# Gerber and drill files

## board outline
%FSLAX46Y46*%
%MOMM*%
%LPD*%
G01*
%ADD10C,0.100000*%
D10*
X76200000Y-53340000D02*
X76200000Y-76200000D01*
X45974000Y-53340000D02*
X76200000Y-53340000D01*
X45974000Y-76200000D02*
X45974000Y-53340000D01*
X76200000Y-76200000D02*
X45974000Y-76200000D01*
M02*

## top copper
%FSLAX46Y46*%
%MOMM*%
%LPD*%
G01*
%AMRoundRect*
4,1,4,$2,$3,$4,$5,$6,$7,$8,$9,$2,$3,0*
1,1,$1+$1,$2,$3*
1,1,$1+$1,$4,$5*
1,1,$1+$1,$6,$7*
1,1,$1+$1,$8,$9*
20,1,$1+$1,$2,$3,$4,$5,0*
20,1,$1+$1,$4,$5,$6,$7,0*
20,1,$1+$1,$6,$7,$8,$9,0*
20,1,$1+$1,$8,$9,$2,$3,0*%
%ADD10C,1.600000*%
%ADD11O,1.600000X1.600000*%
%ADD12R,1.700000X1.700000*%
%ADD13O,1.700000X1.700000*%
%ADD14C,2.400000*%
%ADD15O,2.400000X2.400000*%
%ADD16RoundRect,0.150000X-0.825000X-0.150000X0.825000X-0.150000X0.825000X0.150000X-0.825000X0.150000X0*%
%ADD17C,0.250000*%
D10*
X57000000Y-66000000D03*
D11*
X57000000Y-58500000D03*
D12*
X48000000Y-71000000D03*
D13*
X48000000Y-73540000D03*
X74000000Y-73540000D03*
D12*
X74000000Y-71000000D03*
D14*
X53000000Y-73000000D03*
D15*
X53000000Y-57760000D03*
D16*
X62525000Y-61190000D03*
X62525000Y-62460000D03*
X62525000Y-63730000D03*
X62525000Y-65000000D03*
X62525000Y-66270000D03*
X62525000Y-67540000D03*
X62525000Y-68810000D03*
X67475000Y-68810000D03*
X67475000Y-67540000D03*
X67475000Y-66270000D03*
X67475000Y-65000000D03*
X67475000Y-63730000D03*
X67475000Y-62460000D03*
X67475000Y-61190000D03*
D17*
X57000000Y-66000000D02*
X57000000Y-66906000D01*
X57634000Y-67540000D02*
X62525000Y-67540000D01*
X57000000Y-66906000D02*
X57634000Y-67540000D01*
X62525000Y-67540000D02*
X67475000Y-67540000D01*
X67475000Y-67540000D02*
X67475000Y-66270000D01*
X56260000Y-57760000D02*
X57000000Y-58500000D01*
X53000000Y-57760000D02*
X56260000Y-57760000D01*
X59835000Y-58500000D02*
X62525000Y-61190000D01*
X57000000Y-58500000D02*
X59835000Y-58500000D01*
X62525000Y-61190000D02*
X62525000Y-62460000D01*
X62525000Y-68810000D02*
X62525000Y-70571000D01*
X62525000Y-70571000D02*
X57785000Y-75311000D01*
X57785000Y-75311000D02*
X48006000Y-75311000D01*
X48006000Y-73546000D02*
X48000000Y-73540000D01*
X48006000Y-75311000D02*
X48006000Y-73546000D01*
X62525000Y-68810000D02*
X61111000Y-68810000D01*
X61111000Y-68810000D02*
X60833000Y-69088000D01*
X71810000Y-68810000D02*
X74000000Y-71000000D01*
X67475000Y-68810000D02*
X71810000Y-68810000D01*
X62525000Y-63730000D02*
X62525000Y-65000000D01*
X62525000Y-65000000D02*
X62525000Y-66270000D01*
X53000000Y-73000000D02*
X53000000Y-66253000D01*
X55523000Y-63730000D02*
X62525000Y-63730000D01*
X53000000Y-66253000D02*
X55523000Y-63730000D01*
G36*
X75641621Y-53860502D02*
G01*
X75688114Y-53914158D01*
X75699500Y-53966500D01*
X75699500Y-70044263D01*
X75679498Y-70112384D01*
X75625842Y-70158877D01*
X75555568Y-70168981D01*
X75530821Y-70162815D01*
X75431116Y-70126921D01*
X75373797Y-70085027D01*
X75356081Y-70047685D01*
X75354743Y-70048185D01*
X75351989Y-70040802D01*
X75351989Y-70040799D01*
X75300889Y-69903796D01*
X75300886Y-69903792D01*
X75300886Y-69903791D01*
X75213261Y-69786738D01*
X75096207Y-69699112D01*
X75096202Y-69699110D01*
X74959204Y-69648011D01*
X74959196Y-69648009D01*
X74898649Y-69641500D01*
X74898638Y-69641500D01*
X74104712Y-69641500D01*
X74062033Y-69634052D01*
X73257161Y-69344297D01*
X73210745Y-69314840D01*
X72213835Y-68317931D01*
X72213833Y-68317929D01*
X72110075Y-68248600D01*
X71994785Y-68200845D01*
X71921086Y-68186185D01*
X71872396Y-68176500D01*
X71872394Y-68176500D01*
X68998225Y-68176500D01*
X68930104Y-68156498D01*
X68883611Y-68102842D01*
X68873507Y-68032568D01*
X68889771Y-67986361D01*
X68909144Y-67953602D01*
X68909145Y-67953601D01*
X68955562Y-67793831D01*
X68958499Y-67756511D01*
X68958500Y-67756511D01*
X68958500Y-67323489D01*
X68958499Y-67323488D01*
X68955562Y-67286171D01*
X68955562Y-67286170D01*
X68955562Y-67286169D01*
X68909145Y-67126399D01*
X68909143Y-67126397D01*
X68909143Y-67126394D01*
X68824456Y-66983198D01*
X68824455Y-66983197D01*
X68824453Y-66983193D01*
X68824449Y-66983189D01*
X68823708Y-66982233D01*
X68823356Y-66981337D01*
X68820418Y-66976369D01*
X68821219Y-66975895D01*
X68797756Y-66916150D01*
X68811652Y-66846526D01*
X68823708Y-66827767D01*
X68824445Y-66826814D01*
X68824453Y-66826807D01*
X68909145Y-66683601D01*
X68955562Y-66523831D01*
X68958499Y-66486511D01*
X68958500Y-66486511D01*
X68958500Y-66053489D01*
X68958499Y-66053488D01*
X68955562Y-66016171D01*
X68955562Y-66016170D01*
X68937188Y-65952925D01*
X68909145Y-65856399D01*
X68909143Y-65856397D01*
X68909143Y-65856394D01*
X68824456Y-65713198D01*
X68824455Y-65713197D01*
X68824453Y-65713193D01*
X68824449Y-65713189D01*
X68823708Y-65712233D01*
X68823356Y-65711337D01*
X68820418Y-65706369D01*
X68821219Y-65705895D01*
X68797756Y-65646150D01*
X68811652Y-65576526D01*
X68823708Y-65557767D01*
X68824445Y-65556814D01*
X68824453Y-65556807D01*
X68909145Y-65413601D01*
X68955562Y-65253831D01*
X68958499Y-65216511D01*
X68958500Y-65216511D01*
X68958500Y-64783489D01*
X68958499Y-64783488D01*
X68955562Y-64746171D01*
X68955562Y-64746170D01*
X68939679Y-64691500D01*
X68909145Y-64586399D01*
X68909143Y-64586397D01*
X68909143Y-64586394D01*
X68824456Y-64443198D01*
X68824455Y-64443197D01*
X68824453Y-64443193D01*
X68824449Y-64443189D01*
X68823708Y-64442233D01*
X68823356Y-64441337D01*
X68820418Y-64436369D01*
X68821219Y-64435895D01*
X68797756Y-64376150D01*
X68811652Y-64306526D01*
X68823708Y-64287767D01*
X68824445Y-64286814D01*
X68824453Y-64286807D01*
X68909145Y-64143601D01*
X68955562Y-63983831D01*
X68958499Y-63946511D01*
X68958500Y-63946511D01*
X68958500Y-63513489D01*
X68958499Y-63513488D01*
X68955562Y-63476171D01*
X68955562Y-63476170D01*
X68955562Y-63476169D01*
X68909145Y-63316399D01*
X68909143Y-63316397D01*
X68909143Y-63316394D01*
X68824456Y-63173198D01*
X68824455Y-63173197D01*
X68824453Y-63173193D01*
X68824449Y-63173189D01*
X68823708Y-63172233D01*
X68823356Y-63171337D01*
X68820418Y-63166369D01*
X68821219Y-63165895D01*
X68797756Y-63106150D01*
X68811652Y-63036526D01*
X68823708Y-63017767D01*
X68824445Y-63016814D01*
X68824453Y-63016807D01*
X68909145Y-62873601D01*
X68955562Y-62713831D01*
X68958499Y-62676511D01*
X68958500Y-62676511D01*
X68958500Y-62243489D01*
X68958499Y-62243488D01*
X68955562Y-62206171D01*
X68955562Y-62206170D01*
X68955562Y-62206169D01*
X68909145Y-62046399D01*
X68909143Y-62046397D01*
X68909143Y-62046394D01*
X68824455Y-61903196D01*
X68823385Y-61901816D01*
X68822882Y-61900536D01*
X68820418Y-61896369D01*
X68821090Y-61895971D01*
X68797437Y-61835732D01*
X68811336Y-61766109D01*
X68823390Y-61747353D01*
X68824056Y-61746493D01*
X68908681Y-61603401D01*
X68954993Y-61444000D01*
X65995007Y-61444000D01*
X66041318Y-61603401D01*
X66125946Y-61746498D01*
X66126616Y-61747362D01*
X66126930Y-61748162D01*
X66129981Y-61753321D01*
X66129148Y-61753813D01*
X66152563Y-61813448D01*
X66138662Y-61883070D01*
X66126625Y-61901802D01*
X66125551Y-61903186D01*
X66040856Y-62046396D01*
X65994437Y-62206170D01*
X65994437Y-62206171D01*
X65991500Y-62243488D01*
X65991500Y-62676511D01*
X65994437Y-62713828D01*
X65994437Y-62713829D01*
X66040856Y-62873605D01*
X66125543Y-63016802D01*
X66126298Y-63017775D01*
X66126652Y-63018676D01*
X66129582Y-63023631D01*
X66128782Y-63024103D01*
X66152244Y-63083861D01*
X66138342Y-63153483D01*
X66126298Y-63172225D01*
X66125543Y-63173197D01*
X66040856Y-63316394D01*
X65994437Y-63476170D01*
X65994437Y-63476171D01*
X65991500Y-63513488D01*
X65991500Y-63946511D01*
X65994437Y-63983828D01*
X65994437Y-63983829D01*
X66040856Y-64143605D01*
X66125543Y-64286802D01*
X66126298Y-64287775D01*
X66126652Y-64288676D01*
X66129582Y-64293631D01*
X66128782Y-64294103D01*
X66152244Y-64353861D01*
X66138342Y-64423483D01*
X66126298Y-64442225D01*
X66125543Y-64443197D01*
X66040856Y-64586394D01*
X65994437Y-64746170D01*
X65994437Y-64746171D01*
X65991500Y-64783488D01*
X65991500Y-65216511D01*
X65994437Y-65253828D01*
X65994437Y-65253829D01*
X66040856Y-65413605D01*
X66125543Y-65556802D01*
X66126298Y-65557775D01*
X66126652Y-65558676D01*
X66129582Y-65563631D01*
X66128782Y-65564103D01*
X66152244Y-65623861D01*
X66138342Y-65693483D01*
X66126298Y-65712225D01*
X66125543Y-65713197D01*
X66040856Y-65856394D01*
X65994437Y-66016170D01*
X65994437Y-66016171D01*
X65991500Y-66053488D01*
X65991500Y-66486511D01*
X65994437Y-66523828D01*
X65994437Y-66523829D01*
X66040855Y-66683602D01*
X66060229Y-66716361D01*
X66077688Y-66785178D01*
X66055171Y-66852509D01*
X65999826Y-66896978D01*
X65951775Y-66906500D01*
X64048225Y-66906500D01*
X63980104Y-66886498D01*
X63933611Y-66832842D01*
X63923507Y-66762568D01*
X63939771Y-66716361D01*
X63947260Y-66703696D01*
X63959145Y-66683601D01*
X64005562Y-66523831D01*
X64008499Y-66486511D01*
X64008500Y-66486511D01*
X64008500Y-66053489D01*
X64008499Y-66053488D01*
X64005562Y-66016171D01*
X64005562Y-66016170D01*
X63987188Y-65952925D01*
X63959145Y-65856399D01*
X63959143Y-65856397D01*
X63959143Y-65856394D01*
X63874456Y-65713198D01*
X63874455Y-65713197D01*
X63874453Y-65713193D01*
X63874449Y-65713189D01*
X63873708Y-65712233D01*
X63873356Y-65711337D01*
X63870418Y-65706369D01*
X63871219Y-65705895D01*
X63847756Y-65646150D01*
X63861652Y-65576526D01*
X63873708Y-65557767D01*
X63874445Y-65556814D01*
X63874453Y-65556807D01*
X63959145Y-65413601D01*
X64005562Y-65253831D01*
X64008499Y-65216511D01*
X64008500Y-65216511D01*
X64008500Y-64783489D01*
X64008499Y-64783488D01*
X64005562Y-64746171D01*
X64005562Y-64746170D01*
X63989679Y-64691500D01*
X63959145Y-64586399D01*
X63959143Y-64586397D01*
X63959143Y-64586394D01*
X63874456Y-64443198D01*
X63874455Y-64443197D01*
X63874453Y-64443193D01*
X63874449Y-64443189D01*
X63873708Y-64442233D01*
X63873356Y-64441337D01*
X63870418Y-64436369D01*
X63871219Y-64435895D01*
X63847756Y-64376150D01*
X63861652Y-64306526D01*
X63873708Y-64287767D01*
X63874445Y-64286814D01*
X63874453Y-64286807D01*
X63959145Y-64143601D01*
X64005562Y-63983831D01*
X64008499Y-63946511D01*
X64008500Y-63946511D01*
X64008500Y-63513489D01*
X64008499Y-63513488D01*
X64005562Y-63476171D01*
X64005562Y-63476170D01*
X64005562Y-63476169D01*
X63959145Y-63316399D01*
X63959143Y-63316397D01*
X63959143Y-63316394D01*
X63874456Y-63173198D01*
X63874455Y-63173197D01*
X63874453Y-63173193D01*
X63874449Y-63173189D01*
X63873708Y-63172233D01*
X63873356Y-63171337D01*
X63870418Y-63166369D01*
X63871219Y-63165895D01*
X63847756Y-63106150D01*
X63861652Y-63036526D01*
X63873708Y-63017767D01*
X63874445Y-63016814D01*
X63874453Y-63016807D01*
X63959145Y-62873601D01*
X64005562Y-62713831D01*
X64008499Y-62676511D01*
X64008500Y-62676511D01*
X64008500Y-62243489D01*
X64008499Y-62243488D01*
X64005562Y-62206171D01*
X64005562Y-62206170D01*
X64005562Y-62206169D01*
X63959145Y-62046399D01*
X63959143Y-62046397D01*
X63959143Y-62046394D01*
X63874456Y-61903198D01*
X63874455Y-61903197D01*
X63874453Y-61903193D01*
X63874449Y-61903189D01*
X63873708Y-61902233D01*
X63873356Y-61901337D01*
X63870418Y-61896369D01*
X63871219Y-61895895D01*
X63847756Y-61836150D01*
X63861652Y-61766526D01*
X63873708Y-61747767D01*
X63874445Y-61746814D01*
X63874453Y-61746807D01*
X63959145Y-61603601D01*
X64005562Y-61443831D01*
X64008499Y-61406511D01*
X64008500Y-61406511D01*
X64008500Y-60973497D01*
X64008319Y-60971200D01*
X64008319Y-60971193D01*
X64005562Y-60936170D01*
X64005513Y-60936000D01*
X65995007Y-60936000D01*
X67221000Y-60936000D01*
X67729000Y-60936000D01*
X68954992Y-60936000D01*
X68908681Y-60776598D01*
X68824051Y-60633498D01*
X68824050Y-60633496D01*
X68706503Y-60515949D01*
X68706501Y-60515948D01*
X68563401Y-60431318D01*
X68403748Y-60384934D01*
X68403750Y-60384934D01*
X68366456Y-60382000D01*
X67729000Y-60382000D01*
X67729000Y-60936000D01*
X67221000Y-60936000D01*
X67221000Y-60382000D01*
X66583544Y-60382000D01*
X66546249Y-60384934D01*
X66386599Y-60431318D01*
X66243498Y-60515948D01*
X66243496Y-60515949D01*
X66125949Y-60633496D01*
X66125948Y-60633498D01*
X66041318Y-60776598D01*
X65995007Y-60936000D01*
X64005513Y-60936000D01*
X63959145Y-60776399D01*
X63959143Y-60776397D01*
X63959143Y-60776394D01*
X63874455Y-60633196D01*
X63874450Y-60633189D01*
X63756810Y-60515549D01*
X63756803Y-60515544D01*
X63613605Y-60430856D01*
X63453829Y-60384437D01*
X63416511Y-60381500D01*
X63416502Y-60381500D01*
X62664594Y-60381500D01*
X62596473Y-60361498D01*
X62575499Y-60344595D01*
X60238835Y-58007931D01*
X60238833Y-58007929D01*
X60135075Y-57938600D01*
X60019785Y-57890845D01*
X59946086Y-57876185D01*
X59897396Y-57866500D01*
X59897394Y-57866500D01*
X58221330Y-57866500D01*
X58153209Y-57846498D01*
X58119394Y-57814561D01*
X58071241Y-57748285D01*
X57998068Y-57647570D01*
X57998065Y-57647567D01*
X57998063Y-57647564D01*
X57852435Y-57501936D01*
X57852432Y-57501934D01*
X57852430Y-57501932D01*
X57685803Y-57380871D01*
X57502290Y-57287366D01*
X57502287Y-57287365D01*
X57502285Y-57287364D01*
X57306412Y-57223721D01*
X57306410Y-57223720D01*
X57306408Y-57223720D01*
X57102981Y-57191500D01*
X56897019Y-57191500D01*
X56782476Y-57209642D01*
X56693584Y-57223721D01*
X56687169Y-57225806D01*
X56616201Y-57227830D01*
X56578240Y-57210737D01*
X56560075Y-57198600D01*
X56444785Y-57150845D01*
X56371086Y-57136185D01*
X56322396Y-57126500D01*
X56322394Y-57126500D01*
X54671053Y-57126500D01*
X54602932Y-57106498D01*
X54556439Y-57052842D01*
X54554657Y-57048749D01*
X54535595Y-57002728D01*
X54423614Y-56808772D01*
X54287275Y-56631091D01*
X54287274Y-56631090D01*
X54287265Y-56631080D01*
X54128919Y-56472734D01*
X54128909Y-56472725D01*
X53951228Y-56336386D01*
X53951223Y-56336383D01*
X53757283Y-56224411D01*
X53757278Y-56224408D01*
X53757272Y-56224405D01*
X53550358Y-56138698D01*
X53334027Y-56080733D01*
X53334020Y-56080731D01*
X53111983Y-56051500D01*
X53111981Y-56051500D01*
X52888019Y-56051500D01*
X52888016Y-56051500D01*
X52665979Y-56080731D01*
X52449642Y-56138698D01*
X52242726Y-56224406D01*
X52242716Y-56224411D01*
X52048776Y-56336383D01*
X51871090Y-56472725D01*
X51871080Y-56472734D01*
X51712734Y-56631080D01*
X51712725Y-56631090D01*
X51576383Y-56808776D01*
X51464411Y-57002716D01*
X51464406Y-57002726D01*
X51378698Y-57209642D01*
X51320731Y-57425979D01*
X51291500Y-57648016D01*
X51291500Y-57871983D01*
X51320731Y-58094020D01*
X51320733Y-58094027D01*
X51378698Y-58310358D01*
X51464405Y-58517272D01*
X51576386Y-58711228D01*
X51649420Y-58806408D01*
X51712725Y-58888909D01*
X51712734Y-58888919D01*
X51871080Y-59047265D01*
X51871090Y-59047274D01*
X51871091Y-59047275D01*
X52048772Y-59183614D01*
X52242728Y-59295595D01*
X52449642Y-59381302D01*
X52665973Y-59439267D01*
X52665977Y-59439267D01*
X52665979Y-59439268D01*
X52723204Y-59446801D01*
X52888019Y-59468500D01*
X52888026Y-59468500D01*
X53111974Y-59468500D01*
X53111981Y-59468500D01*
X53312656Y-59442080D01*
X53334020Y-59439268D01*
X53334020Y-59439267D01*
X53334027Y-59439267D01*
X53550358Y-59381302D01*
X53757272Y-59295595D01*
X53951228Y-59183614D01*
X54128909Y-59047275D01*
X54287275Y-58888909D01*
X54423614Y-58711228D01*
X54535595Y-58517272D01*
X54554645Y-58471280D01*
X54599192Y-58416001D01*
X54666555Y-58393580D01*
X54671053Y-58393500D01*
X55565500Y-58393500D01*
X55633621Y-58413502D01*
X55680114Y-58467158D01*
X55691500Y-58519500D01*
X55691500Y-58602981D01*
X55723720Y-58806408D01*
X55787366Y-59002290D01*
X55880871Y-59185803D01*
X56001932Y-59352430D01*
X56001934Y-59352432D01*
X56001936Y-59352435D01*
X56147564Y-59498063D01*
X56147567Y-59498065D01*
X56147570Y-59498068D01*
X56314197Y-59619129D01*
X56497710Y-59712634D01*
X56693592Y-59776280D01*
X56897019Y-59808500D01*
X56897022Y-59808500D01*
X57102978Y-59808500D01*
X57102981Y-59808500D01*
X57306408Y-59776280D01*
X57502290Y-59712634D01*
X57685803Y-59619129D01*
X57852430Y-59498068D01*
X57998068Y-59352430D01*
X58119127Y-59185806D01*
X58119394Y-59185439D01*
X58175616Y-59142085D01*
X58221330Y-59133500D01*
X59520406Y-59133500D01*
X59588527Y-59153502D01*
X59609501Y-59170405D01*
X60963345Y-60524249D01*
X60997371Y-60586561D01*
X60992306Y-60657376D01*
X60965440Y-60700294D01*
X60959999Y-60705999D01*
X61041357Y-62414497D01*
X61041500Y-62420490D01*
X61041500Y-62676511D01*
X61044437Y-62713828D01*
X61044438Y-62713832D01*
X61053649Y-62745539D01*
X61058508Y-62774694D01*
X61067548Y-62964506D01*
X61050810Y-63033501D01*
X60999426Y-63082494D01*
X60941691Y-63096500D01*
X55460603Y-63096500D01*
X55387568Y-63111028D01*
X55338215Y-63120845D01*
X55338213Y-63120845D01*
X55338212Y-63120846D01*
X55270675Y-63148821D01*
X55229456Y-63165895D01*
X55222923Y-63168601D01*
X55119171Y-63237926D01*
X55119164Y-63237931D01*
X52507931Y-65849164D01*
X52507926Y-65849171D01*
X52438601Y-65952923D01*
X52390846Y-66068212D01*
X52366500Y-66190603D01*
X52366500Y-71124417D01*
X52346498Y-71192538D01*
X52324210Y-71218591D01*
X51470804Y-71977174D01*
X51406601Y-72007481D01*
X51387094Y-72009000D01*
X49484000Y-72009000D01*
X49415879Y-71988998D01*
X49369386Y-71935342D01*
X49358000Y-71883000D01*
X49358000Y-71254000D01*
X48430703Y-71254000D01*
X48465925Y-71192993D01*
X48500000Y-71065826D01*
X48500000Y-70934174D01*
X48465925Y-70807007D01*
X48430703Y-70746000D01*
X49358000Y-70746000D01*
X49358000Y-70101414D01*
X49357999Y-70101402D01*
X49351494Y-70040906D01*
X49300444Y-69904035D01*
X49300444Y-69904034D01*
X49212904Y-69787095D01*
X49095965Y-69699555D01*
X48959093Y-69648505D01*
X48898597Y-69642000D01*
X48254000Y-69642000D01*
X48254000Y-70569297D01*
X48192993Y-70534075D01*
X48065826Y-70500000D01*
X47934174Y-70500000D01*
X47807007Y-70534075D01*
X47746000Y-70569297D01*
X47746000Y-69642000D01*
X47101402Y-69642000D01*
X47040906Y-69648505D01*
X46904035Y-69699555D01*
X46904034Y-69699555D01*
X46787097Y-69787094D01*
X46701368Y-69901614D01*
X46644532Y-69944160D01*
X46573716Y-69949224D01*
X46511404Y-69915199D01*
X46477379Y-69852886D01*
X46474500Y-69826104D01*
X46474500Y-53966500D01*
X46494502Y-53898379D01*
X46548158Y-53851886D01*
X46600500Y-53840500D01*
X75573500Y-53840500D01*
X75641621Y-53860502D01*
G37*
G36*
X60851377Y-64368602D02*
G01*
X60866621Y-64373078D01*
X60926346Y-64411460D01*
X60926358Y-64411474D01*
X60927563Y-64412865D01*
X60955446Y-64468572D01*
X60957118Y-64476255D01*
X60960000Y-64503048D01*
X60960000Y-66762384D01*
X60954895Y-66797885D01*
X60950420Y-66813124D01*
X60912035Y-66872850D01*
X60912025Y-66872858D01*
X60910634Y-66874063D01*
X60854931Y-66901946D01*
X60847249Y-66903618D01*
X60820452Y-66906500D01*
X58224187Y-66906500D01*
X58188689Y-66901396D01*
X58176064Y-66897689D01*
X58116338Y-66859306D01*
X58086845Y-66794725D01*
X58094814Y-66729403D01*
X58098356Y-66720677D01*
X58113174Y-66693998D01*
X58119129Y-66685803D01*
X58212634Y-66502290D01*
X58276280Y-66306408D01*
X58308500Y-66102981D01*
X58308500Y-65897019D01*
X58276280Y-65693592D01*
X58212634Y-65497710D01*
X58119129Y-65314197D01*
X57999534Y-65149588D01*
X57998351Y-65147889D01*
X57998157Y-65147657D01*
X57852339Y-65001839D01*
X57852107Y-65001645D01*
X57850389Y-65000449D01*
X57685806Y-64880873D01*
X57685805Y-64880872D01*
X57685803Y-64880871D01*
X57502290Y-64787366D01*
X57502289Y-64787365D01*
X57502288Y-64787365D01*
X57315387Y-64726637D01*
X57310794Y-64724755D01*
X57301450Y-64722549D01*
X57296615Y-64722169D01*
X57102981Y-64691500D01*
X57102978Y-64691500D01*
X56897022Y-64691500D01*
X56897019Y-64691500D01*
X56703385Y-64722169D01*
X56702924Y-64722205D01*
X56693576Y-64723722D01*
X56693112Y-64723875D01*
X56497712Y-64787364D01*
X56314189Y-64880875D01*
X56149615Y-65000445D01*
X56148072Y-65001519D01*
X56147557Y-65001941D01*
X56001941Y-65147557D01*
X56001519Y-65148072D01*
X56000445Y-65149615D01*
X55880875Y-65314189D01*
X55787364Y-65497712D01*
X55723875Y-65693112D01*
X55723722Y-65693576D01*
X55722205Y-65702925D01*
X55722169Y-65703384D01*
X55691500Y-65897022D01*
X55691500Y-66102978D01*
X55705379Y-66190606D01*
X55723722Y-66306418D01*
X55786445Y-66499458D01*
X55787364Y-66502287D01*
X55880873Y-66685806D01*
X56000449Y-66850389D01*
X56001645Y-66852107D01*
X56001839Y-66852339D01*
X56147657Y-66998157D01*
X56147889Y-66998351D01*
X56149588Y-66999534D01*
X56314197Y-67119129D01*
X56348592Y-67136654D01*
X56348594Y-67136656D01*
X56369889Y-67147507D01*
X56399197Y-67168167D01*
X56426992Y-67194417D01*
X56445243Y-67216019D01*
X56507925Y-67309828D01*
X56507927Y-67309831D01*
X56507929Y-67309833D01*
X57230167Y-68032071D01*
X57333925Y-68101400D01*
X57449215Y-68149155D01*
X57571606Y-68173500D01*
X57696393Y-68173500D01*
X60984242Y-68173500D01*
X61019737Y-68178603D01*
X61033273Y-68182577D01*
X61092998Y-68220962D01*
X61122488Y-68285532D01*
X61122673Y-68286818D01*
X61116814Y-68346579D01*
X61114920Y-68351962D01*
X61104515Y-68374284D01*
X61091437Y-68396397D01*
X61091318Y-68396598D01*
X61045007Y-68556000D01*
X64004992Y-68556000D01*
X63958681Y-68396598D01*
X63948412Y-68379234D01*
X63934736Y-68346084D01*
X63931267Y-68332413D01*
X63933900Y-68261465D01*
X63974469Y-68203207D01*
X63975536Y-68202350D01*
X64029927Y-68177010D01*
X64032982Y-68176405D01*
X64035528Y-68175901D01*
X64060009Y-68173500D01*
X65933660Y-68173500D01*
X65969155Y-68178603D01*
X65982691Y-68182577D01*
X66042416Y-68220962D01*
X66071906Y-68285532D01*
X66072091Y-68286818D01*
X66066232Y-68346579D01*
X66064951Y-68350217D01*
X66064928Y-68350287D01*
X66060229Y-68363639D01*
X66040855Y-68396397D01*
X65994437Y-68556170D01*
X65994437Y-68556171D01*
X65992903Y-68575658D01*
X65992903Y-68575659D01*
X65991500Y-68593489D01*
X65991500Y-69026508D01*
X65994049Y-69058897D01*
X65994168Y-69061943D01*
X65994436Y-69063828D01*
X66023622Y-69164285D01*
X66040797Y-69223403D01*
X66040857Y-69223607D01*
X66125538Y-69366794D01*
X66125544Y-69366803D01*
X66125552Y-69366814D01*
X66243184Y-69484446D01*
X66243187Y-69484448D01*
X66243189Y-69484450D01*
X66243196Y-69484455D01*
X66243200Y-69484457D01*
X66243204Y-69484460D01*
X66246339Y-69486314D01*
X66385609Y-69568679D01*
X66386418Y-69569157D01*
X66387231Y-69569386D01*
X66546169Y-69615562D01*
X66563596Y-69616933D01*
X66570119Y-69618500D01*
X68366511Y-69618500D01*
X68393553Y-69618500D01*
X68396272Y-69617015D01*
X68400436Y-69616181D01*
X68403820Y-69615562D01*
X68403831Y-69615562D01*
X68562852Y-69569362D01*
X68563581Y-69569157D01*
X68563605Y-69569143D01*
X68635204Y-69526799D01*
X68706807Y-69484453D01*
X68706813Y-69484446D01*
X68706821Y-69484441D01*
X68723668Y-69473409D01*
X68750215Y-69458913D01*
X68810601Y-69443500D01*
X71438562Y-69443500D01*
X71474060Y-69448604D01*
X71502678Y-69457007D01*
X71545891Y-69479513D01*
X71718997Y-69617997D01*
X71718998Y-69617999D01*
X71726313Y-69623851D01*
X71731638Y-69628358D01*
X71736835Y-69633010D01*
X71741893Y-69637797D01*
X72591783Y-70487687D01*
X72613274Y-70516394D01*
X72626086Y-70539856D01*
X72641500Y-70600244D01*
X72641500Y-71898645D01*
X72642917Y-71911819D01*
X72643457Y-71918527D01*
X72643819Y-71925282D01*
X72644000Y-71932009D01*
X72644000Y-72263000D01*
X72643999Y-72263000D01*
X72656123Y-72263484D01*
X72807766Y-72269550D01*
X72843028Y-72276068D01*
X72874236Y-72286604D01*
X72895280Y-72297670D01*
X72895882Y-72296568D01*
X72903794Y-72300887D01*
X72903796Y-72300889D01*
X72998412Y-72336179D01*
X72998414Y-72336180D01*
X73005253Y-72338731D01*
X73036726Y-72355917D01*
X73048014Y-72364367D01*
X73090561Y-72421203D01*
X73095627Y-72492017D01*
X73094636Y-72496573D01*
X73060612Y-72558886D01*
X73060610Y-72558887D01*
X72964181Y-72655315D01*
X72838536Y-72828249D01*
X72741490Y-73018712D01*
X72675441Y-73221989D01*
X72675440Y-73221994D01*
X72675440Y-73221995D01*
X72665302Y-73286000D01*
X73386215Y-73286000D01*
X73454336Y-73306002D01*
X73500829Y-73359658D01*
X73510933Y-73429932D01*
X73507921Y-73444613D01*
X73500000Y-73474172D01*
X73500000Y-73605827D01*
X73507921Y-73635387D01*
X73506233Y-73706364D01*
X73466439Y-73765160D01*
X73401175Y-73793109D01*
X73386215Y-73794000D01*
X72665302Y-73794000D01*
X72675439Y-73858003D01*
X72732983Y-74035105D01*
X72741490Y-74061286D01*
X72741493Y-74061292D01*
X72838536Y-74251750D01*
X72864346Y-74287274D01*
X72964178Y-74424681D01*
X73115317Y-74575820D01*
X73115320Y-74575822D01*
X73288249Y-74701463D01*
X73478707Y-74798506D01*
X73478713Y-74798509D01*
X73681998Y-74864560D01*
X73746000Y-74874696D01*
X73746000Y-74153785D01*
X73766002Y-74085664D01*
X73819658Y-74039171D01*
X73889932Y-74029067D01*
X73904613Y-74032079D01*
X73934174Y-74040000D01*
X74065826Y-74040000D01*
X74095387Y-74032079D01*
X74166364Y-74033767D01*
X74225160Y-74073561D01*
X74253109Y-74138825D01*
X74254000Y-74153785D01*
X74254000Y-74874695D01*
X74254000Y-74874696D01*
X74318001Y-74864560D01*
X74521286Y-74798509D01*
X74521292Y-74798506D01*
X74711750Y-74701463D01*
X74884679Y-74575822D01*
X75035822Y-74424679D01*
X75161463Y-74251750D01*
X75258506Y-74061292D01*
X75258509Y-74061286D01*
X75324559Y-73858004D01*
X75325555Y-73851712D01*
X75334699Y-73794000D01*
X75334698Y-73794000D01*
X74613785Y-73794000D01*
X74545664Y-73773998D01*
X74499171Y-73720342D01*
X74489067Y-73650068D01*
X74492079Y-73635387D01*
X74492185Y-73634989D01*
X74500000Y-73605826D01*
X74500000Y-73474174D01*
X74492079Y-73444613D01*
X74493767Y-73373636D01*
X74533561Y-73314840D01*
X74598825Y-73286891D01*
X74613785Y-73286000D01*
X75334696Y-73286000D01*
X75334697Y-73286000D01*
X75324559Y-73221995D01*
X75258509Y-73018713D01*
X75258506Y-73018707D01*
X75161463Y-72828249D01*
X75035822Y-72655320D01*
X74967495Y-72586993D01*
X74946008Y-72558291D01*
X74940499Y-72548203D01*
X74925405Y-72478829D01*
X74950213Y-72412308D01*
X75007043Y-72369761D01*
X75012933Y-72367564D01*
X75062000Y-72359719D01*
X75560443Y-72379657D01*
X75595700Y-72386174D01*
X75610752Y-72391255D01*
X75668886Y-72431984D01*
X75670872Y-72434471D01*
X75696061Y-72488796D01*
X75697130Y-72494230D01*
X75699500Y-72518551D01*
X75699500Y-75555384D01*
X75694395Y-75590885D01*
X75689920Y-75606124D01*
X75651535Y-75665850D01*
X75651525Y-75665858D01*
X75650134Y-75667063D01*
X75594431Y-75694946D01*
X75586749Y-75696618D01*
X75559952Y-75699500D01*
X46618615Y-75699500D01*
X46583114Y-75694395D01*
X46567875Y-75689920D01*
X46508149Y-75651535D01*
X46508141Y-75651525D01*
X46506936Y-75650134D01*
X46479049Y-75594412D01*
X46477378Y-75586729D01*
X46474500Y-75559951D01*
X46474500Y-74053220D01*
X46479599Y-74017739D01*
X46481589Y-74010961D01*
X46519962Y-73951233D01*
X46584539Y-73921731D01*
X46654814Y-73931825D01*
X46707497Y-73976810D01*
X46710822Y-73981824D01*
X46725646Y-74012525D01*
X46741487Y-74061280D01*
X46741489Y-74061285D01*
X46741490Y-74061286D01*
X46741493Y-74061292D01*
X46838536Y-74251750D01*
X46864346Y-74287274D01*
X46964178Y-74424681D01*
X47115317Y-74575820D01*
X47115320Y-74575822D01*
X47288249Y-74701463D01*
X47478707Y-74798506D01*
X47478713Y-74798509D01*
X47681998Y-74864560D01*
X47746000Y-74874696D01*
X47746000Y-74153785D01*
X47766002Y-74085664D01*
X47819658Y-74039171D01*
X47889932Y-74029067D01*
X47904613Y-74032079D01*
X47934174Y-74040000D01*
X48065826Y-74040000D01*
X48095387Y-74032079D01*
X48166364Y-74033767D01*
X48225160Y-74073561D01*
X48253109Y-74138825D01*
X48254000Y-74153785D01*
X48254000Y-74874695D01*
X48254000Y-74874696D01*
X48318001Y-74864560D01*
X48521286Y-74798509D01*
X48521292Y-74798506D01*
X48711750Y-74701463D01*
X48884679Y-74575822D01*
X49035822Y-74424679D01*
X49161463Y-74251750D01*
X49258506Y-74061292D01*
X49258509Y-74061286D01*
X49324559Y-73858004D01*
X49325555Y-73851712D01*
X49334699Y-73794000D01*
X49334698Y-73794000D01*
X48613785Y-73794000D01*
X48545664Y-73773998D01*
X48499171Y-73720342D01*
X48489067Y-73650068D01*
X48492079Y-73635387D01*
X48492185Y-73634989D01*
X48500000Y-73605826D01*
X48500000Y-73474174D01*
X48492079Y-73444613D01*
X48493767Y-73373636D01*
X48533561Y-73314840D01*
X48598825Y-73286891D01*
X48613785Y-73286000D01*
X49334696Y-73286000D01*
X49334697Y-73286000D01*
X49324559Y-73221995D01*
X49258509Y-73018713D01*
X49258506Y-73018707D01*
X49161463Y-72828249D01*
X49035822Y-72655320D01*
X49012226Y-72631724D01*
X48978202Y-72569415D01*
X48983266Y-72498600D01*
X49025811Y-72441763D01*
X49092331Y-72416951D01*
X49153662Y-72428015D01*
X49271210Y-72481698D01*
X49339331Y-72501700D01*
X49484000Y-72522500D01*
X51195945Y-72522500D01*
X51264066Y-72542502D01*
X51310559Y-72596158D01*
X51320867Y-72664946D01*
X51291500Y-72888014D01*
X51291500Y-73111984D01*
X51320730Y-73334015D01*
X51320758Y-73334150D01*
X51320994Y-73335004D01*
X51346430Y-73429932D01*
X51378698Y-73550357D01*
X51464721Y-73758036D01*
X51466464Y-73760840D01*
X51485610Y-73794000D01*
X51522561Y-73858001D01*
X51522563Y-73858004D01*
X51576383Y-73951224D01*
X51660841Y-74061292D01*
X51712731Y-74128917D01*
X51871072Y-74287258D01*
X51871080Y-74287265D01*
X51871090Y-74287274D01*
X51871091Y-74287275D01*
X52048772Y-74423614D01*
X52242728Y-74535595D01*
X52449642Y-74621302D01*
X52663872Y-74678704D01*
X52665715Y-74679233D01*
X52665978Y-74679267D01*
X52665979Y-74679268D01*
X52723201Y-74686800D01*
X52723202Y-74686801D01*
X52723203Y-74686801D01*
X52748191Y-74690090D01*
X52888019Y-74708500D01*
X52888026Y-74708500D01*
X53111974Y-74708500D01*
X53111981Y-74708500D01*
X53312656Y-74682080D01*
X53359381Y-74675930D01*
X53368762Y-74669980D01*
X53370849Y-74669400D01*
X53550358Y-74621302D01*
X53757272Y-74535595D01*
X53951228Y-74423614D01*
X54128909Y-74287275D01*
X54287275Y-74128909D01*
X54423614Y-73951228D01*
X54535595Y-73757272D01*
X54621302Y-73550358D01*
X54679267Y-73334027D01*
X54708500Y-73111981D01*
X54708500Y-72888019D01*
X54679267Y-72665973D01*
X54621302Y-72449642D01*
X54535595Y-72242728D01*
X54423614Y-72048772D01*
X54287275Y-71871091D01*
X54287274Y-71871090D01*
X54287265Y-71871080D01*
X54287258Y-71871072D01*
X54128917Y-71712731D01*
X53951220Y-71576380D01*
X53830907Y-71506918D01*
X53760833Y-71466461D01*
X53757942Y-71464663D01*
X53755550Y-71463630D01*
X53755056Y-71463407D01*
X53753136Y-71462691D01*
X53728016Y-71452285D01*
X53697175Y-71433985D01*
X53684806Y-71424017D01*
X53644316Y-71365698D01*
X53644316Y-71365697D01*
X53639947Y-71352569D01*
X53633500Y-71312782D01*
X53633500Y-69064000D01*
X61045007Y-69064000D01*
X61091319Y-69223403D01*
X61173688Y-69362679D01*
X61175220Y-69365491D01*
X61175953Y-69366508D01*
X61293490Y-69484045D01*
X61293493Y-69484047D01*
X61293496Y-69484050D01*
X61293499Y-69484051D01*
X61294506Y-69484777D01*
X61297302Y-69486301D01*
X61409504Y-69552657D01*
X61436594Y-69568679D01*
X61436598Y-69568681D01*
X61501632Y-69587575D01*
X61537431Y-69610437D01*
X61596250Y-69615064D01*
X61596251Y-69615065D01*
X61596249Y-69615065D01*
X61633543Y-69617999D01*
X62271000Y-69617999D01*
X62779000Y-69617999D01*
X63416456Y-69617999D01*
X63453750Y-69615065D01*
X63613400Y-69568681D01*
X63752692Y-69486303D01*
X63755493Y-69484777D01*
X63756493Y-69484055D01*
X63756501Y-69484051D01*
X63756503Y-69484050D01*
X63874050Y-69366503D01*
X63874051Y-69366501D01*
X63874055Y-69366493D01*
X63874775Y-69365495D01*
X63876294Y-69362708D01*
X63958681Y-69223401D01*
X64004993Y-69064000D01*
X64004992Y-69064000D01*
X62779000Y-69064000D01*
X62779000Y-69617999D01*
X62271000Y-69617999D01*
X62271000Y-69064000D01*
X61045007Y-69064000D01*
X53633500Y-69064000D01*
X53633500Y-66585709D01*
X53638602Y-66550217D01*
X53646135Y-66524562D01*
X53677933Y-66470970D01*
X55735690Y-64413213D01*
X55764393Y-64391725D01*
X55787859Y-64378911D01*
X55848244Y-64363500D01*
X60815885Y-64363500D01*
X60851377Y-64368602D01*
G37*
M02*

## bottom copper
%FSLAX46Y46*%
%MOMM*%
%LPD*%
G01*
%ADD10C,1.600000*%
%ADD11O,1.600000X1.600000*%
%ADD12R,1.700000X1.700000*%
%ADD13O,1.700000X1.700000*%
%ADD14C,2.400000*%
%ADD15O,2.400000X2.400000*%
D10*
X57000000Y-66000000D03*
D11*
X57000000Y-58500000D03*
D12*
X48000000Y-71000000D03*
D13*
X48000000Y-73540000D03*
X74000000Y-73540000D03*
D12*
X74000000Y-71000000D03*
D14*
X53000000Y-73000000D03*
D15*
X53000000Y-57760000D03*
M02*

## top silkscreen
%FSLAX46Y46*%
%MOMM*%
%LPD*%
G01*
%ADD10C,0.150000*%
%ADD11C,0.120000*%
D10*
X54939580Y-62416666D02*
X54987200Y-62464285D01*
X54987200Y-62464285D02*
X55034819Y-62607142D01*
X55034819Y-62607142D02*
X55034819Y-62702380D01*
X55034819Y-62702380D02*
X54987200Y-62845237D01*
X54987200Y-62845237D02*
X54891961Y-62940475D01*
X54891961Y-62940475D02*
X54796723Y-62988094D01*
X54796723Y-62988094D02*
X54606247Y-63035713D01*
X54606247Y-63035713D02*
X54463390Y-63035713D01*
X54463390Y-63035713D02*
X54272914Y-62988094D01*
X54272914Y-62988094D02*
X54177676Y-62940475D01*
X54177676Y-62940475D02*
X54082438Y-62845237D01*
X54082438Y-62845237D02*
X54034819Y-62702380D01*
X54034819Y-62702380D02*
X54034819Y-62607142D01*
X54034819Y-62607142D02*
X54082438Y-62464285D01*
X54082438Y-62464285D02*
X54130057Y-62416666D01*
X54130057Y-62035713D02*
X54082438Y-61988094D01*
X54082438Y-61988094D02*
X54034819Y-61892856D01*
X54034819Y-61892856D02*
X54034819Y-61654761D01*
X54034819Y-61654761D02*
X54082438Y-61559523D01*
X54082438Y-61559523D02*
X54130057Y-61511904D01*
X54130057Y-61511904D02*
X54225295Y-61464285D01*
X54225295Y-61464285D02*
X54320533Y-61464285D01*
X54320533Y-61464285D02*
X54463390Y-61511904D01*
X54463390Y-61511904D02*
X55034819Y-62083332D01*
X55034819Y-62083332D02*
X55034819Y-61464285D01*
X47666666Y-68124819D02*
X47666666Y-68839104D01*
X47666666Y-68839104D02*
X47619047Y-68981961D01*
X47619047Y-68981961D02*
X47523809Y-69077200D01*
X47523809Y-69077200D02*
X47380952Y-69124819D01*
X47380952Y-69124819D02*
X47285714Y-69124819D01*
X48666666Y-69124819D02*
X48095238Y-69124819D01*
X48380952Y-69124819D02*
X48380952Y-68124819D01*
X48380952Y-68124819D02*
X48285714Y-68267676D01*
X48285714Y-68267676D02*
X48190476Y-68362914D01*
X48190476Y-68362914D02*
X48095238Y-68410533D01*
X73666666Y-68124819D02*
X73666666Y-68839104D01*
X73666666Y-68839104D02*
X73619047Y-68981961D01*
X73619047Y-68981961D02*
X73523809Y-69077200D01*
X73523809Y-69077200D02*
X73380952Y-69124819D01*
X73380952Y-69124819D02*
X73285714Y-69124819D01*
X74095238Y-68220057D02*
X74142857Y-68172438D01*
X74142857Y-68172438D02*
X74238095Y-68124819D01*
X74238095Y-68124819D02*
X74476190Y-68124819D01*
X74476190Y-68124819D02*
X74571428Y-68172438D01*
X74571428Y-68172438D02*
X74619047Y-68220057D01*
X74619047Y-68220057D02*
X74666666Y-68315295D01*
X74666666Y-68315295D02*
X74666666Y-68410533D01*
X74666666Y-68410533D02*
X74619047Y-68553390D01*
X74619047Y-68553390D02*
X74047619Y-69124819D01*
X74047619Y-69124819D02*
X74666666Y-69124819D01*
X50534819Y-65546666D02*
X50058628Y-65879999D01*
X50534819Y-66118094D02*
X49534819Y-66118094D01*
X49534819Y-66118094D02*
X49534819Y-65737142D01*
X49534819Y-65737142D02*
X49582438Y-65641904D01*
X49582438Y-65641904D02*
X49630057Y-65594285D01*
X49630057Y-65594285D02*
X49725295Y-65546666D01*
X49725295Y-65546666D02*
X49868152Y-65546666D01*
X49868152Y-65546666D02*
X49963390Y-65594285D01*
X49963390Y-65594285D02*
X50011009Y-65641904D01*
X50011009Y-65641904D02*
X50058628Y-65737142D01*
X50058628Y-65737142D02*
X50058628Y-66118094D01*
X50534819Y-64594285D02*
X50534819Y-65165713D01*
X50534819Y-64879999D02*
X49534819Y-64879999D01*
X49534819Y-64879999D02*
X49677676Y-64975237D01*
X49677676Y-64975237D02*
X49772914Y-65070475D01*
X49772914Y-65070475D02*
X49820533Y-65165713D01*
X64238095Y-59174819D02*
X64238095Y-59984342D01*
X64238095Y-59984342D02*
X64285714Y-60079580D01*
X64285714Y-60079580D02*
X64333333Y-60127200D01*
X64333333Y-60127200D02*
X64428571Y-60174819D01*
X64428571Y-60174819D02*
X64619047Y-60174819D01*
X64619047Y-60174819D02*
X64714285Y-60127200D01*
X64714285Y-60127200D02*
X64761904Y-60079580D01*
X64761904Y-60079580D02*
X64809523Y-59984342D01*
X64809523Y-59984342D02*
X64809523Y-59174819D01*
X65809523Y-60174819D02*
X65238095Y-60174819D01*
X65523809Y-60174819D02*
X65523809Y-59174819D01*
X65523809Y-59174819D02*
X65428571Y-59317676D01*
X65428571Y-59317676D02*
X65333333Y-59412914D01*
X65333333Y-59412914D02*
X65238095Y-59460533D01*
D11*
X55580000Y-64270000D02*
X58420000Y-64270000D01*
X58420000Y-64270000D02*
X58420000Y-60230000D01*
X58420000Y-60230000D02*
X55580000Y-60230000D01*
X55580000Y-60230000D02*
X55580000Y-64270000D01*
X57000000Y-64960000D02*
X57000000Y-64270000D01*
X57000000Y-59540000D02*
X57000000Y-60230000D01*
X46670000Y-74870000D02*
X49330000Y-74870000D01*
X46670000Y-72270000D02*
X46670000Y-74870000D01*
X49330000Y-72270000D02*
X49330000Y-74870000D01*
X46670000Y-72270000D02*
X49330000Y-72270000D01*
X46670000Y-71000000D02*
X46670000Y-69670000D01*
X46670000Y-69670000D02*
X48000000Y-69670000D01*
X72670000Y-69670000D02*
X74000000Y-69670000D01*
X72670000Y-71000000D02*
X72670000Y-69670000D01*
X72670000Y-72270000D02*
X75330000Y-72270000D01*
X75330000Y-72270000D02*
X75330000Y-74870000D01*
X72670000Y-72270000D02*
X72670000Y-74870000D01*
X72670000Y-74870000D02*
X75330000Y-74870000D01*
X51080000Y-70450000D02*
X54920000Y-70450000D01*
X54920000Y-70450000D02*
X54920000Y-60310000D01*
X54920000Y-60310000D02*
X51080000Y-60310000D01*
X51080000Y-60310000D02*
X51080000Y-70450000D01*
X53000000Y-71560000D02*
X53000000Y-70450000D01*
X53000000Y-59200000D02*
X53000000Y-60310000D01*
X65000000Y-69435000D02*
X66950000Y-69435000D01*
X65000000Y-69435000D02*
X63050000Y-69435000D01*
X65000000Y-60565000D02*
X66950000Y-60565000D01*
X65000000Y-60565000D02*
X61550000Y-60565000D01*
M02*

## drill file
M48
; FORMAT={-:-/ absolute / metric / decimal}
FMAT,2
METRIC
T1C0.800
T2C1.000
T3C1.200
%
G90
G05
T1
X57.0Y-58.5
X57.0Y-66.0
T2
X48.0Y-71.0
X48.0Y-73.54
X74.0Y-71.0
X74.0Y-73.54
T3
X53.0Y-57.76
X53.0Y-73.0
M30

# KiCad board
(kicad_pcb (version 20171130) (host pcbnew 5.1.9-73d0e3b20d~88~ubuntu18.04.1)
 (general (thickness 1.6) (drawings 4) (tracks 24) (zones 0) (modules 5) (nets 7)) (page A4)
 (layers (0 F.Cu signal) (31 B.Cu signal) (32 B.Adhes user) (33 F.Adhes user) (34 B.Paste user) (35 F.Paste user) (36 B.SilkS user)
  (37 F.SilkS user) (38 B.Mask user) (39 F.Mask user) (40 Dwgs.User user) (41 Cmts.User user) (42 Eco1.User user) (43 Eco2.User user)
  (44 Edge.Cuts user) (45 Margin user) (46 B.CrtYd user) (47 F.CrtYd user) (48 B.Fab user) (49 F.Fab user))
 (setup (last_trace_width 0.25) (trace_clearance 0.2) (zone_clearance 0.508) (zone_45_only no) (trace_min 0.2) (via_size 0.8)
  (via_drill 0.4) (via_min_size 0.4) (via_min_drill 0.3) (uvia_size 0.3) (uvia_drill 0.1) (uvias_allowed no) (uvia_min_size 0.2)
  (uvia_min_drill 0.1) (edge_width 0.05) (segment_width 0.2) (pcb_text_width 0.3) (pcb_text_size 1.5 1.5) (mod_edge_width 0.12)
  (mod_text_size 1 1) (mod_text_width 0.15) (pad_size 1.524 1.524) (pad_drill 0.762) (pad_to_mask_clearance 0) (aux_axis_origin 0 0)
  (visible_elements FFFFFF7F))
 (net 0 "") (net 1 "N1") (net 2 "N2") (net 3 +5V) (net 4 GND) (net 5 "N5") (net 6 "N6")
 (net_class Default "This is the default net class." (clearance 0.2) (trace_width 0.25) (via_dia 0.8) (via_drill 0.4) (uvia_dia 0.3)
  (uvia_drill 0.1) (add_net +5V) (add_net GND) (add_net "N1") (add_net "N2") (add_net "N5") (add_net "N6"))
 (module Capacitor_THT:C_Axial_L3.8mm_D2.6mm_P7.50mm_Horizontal (layer F.Cu) (at 57 66 90)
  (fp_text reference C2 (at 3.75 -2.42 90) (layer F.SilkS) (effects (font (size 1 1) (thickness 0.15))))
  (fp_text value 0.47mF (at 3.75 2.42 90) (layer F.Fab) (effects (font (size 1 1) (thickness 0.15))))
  (fp_line (start 1.73 -1.42) (end 1.73 1.42) (layer F.SilkS) (width 0.12))
  (fp_line (start 1.73 1.42) (end 5.77 1.42) (layer F.SilkS) (width 0.12))
  (fp_line (start 5.77 1.42) (end 5.77 -1.42) (layer F.SilkS) (width 0.12))
  (fp_line (start 5.77 -1.42) (end 1.73 -1.42) (layer F.SilkS) (width 0.12))
  (fp_line (start 1.04 0) (end 1.73 0) (layer F.SilkS) (width 0.12))
  (fp_line (start 6.46 0) (end 5.77 0) (layer F.SilkS) (width 0.12))
  (pad 1 thru_hole circle (at 0 0 90) (size 1.6 1.6) (drill 0.8) (layers *.Cu *.Mask) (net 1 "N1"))
  (pad 2 thru_hole oval (at 7.5 0 90) (size 1.6 1.6) (drill 0.8) (layers *.Cu *.Mask) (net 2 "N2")))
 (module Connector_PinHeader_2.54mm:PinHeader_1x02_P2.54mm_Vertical (layer F.Cu) (at 48 71)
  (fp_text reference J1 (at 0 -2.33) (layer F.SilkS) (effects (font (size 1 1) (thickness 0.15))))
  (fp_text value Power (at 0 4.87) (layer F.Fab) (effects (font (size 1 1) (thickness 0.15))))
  (fp_line (start -1.33 3.87) (end 1.33 3.87) (layer F.SilkS) (width 0.12))
  (fp_line (start -1.33 1.27) (end -1.33 3.87) (layer F.SilkS) (width 0.12))
  (fp_line (start 1.33 1.27) (end 1.33 3.87) (layer F.SilkS) (width 0.12))
  (fp_line (start -1.33 1.27) (end 1.33 1.27) (layer F.SilkS) (width 0.12))
  (fp_line (start -1.33 0) (end -1.33 -1.33) (layer F.SilkS) (width 0.12))
  (fp_line (start -1.33 -1.33) (end 0 -1.33) (layer F.SilkS) (width 0.12))
  (pad 1 thru_hole rect (at 0 0) (size 1.7 1.7) (drill 1) (layers *.Cu *.Mask) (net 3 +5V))
  (pad 2 thru_hole oval (at 0 2.54) (size 1.7 1.7) (drill 1) (layers *.Cu *.Mask) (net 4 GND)))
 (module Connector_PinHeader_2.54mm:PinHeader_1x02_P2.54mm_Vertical (layer F.Cu) (at 74 71)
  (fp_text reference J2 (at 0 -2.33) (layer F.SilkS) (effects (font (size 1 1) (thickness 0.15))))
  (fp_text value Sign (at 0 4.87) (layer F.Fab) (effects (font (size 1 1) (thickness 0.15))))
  (fp_line (start -1.33 -1.33) (end 0 -1.33) (layer F.SilkS) (width 0.12))
  (fp_line (start -1.33 0) (end -1.33 -1.33) (layer F.SilkS) (width 0.12))
  (fp_line (start -1.33 1.27) (end 1.33 1.27) (layer F.SilkS) (width 0.12))
  (fp_line (start 1.33 1.27) (end 1.33 3.87) (layer F.SilkS) (width 0.12))
  (fp_line (start -1.33 1.27) (end -1.33 3.87) (layer F.SilkS) (width 0.12))
  (fp_line (start -1.33 3.87) (end 1.33 3.87) (layer F.SilkS) (width 0.12))
  (pad 2 thru_hole oval (at 0 2.54) (size 1.7 1.7) (drill 1) (layers *.Cu *.Mask) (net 4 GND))
  (pad 1 thru_hole rect (at 0 0) (size 1.7 1.7) (drill 1) (layers *.Cu *.Mask) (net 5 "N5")))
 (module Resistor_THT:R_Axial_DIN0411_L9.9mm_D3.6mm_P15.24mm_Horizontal (layer F.Cu) (at 53 73 90)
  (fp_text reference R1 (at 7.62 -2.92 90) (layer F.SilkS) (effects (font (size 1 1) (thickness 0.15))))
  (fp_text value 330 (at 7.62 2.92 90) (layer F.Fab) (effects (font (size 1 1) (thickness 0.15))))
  (fp_line (start 2.55 -1.92) (end 2.55 1.92) (layer F.SilkS) (width 0.12))
  (fp_line (start 2.55 1.92) (end 12.69 1.92) (layer F.SilkS) (width 0.12))
  (fp_line (start 12.69 1.92) (end 12.69 -1.92) (layer F.SilkS) (width 0.12))
  (fp_line (start 12.69 -1.92) (end 2.55 -1.92) (layer F.SilkS) (width 0.12))
  (fp_line (start 1.44 0) (end 2.55 0) (layer F.SilkS) (width 0.12))
  (fp_line (start 13.8 0) (end 12.69 0) (layer F.SilkS) (width 0.12))
  (pad 1 thru_hole circle (at 0 0 90) (size 2.4 2.4) (drill 1.2) (layers *.Cu *.Mask) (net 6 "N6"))
  (pad 2 thru_hole oval (at 15.24 0 90) (size 2.4 2.4) (drill 1.2) (layers *.Cu *.Mask) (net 2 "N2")))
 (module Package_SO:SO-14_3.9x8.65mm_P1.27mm (layer F.Cu) (at 65 65)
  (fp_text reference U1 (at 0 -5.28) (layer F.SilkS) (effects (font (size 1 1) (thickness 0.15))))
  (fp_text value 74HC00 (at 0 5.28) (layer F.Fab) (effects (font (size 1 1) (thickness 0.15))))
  (fp_line (start 0 4.435) (end 1.95 4.435) (layer F.SilkS) (width 0.12))
  (fp_line (start 0 4.435) (end -1.95 4.435) (layer F.SilkS) (width 0.12))
  (fp_line (start 0 -4.435) (end 1.95 -4.435) (layer F.SilkS) (width 0.12))
  (fp_line (start 0 -4.435) (end -3.45 -4.435) (layer F.SilkS) (width 0.12))
  (pad 1 smd roundrect (at -2.475 -3.81) (size 1.95 0.6) (layers F.Cu F.Paste F.Mask) (roundrect_rratio 0.25) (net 2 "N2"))
  (pad 2 smd roundrect (at -2.475 -2.54) (size 1.95 0.6) (layers F.Cu F.Paste F.Mask) (roundrect_rratio 0.25) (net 2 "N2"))
  (pad 3 smd roundrect (at -2.475 -1.27) (size 1.95 0.6) (layers F.Cu F.Paste F.Mask) (roundrect_rratio 0.25) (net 6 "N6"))
  (pad 4 smd roundrect (at -2.475 0) (size 1.95 0.6) (layers F.Cu F.Paste F.Mask) (roundrect_rratio 0.25) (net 6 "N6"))
  (pad 5 smd roundrect (at -2.475 1.27) (size 1.95 0.6) (layers F.Cu F.Paste F.Mask) (roundrect_rratio 0.25) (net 6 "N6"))
  (pad 6 smd roundrect (at -2.475 2.54) (size 1.95 0.6) (layers F.Cu F.Paste F.Mask) (roundrect_rratio 0.25) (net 1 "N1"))
  (pad 7 smd roundrect (at -2.475 3.81) (size 1.95 0.6) (layers F.Cu F.Paste F.Mask) (roundrect_rratio 0.25) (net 4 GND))
  (pad 8 smd roundrect (at 2.475 3.81) (size 1.95 0.6) (layers F.Cu F.Paste F.Mask) (roundrect_rratio 0.25) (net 5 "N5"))
  (pad 9 smd roundrect (at 2.475 2.54) (size 1.95 0.6) (layers F.Cu F.Paste F.Mask) (roundrect_rratio 0.25) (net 1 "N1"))
  (pad 10 smd roundrect (at 2.475 1.27) (size 1.95 0.6) (layers F.Cu F.Paste F.Mask) (roundrect_rratio 0.25) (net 1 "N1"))
  (pad 11 smd roundrect (at 2.475 0) (size 1.95 0.6) (layers F.Cu F.Paste F.Mask) (roundrect_rratio 0.25))
  (pad 12 smd roundrect (at 2.475 -1.27) (size 1.95 0.6) (layers F.Cu F.Paste F.Mask) (roundrect_rratio 0.25))
  (pad 13 smd roundrect (at 2.475 -2.54) (size 1.95 0.6) (layers F.Cu F.Paste F.Mask) (roundrect_rratio 0.25))
  (pad 14 smd roundrect (at 2.475 -3.81) (size 1.95 0.6) (layers F.Cu F.Paste F.Mask) (roundrect_rratio 0.25) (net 3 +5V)))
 (gr_line (start 76.2 53.34) (end 76.2 76.2) (layer Edge.Cuts) (width 0.1))
 (gr_line (start 45.974 53.34) (end 76.2 53.34) (layer Edge.Cuts) (width 0.1))
 (gr_line (start 45.974 76.2) (end 45.974 53.34) (layer Edge.Cuts) (width 0.1))
 (gr_line (start 76.2 76.2) (end 45.974 76.2) (layer Edge.Cuts) (width 0.1))
 (segment (start 57 66) (end 57 66.906) (width 0.25) (layer F.Cu) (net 1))
 (segment (start 57.634 67.54) (end 62.525 67.54) (width 0.25) (layer F.Cu) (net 1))
 (segment (start 57 66.906) (end 57.634 67.54) (width 0.25) (layer F.Cu) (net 1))
 (segment (start 62.525 67.54) (end 67.475 67.54) (width 0.25) (layer F.Cu) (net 1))
 (segment (start 67.475 67.54) (end 67.475 66.27) (width 0.25) (layer F.Cu) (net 1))
 (segment (start 56.26 57.76) (end 57 58.5) (width 0.25) (layer F.Cu) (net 2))
 (segment (start 53 57.76) (end 56.26 57.76) (width 0.25) (layer F.Cu) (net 2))
 (segment (start 59.835 58.5) (end 62.525 61.19) (width 0.25) (layer F.Cu) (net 2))
 (segment (start 57 58.5) (end 59.835 58.5) (width 0.25) (layer F.Cu) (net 2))
 (segment (start 62.525 61.19) (end 62.525 62.46) (width 0.25) (layer F.Cu) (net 2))
 (segment (start 62.525 68.81) (end 62.525 70.571) (width 0.25) (layer F.Cu) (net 4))
 (segment (start 62.525 70.571) (end 57.785 75.311) (width 0.25) (layer F.Cu) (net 4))
 (segment (start 57.785 75.311) (end 48.006 75.311) (width 0.25) (layer F.Cu) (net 4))
 (segment (start 48.006 73.546) (end 48 73.54) (width 0.25) (layer F.Cu) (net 4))
 (segment (start 48.006 75.311) (end 48.006 73.546) (width 0.25) (layer F.Cu) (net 4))
 (segment (start 62.525 68.81) (end 61.111 68.81) (width 0.25) (layer F.Cu) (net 4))
 (segment (start 61.111 68.81) (end 60.833 69.088) (width 0.25) (layer F.Cu) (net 4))
 (segment (start 71.81 68.81) (end 74 71) (width 0.25) (layer F.Cu) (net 5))
 (segment (start 67.475 68.81) (end 71.81 68.81) (width 0.25) (layer F.Cu) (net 5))
 (segment (start 62.525 63.73) (end 62.525 65) (width 0.25) (layer F.Cu) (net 6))
 (segment (start 62.525 65) (end 62.525 66.27) (width 0.25) (layer F.Cu) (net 6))
 (segment (start 53 73) (end 53 66.253) (width 0.25) (layer F.Cu) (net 6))
 (segment (start 55.523 63.73) (end 62.525 63.73) (width 0.25) (layer F.Cu) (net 6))
 (segment (start 53 66.253) (end 55.523 63.73) (width 0.25) (layer F.Cu) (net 6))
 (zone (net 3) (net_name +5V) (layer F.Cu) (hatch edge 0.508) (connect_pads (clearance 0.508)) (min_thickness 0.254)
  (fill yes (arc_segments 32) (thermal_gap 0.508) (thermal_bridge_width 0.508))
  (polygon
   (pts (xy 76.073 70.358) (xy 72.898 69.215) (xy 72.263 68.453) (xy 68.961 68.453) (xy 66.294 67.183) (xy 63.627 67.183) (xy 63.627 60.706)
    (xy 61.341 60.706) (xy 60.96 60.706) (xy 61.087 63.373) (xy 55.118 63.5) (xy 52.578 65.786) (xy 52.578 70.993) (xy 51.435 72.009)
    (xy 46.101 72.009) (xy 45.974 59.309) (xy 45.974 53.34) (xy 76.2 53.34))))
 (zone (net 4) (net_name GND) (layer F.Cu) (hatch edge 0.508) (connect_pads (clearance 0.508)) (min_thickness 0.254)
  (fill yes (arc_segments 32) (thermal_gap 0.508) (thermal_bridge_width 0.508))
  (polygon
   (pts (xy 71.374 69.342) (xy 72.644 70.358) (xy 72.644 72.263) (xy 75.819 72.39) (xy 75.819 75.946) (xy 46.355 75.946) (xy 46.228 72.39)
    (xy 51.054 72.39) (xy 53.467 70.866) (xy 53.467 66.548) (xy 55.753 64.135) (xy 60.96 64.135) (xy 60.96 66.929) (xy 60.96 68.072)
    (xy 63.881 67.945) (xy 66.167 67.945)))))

